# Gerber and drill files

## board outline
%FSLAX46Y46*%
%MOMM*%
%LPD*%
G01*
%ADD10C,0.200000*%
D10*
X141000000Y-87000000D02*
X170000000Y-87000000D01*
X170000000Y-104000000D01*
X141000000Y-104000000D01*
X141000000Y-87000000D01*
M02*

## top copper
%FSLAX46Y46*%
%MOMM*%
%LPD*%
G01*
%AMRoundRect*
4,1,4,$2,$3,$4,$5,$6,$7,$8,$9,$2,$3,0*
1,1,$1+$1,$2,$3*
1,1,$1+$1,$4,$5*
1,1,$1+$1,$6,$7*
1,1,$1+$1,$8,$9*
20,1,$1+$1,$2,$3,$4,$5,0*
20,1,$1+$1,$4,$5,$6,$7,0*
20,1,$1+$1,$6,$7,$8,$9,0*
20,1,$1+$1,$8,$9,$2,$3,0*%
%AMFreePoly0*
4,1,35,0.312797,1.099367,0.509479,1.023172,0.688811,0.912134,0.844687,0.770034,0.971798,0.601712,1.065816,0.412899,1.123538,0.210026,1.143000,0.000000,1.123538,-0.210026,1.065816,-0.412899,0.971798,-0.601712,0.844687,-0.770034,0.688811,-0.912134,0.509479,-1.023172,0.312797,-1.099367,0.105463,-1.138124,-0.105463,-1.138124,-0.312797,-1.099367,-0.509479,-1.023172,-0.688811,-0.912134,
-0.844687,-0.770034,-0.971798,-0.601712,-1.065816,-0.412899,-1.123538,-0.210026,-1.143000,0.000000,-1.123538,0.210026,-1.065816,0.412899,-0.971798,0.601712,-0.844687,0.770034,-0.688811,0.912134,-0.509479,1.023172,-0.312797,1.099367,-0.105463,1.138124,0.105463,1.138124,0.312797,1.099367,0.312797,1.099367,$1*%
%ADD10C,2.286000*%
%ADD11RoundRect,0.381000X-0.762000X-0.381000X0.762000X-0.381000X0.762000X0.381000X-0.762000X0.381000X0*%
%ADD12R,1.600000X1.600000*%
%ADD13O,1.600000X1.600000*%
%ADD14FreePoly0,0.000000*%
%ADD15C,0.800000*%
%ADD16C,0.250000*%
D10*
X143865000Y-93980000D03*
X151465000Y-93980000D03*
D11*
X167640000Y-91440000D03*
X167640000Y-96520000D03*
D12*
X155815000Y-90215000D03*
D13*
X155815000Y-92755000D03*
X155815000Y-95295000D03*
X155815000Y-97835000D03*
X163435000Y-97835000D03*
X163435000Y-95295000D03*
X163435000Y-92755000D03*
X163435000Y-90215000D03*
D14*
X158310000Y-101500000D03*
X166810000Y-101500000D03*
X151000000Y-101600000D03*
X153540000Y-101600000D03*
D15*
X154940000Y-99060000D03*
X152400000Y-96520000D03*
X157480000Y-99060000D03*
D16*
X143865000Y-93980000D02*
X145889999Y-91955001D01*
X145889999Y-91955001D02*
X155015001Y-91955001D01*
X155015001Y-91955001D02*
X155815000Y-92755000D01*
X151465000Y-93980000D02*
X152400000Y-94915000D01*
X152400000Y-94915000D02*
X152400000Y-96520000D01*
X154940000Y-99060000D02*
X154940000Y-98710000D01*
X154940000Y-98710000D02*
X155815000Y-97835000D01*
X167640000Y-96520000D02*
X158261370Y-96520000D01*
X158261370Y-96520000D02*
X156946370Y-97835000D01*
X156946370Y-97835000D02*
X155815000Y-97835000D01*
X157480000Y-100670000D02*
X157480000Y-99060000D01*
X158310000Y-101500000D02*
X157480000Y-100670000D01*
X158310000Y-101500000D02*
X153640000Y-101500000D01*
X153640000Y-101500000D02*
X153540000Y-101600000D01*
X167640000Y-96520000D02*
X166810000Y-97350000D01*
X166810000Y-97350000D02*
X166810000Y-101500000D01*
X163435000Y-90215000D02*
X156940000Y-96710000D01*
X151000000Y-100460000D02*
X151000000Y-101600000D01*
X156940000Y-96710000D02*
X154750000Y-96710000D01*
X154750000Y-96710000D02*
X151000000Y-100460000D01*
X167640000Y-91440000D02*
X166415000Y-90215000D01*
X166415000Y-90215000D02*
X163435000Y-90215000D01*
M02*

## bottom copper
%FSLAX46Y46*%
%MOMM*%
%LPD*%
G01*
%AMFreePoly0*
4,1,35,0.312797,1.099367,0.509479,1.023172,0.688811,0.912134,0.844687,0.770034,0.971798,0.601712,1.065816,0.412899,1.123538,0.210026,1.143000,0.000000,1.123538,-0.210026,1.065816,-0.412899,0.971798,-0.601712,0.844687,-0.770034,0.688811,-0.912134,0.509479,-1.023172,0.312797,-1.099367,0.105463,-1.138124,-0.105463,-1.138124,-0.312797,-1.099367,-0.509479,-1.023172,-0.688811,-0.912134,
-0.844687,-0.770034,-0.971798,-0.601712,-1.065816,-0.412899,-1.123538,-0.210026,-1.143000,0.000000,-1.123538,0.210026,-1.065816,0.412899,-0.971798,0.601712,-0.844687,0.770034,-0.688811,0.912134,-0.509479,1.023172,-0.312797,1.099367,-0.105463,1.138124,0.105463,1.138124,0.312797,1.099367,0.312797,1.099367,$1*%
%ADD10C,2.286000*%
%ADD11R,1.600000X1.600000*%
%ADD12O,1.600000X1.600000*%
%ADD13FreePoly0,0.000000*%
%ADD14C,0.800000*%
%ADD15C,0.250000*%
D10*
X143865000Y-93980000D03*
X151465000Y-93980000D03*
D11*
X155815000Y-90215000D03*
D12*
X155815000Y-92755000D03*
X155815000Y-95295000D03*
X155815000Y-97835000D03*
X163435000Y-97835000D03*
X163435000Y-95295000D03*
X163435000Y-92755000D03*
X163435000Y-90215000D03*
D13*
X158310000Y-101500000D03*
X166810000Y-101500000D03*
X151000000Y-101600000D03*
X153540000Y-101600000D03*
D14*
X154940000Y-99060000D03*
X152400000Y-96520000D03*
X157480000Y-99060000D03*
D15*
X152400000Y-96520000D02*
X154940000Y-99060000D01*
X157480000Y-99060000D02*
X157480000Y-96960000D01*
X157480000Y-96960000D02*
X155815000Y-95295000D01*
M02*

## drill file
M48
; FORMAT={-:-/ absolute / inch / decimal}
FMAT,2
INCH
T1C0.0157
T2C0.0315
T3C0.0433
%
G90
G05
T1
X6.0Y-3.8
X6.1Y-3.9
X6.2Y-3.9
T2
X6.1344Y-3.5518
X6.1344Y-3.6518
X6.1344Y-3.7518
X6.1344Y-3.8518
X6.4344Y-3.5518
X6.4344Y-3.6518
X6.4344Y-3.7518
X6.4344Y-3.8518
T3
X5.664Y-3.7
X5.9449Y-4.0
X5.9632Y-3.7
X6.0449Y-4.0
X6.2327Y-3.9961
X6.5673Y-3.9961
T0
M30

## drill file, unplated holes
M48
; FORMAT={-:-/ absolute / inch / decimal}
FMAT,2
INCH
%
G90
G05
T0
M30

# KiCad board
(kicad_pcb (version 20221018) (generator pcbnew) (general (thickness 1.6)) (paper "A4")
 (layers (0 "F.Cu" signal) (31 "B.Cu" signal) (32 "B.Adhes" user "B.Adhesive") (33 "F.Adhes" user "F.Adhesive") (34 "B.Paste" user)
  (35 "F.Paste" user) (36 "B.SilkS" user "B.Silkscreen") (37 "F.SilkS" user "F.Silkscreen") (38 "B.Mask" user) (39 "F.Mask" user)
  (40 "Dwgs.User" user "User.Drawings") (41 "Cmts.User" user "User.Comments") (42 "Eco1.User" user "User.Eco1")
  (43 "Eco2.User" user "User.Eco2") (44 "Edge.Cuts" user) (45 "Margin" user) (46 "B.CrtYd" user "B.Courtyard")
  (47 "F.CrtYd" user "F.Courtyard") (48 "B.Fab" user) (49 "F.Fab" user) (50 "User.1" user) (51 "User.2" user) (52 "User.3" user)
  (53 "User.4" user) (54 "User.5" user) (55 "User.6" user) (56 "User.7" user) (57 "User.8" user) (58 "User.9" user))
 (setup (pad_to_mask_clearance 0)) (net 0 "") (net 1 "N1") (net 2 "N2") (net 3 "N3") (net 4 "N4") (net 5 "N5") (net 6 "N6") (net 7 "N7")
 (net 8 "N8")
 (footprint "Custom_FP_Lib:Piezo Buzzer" (layer "F.Cu") (at 143.865 93.98)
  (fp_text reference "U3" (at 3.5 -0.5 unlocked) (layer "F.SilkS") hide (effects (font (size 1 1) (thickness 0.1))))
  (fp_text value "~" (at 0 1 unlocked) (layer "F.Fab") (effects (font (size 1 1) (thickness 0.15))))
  (pad "1" thru_hole circle (at 0 0 90) (size 2.286 2.286) (drill 1.1) (layers "*.Cu" "*.Mask") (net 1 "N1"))
  (pad "2" thru_hole circle (at 7.6 0) (size 2.286 2.286) (drill 1.1) (layers "*.Cu" "*.Mask") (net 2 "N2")))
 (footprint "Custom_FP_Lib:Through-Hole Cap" (layer "F.Cu") (at 151 102.87)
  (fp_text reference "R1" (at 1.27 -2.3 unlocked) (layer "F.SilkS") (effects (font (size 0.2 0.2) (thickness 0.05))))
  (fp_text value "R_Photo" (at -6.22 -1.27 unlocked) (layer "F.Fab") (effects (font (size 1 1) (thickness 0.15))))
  (pad "1" thru_hole custom (at 0 -1.27) (size 2.286 2.286) (drill 1.1) (layers "*.Cu" "*.Mask") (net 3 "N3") (thermal_bridge_angle 45)
   (options (clearance outline) (anchor circle)) (primitives))
  (pad "2" thru_hole custom (at 2.54 -1.27) (size 2.286 2.286) (drill 1.1) (layers "*.Cu" "*.Mask") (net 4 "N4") (thermal_bridge_angle 45)
   (options (clearance outline) (anchor circle)) (primitives)))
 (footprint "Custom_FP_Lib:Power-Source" (layer "F.Cu") (at 165.1 93.98)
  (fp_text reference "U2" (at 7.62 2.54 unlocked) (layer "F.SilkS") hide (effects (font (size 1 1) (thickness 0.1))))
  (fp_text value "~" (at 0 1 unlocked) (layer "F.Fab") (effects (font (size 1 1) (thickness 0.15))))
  (pad "1" smd roundrect (at 2.54 -2.54) (size 2.286 1.524) (layers "F.Cu" "F.Paste" "F.Mask") (roundrect_rratio 0.25) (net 3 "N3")
   (thermal_bridge_angle 45))
  (pad "2" smd roundrect (at 2.54 2.54) (size 2.286 1.524) (layers "F.Cu" "F.Paste" "F.Mask") (roundrect_rratio 0.25) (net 2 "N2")
   (thermal_bridge_angle 45)))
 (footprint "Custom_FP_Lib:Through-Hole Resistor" (layer "F.Cu") (at 157.99 102.77)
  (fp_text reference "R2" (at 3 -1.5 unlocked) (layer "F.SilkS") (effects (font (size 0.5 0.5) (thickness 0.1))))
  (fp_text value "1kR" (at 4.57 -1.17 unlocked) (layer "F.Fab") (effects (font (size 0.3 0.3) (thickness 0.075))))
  (pad "1" thru_hole custom (at 0.32 -1.27) (size 2.286 2.286) (drill 1.1) (layers "*.Cu" "*.Mask") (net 4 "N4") (thermal_bridge_angle 45)
   (options (clearance outline) (anchor circle)) (primitives))
  (pad "2" thru_hole custom (at 8.82 -1.27) (size 2.286 2.286) (drill 1.1) (layers "*.Cu" "*.Mask") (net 2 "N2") (thermal_bridge_angle 45)
   (options (clearance outline) (anchor circle)) (primitives)))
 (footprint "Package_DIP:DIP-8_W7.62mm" (layer "F.Cu") (at 155.815 90.215)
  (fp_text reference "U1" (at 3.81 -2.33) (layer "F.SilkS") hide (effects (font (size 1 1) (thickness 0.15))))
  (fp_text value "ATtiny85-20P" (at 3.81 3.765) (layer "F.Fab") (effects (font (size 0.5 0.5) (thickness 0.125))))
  (pad "1" thru_hole rect (at 0 0) (size 1.6 1.6) (drill 0.8) (layers "*.Cu" "*.Mask") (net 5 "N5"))
  (pad "2" thru_hole oval (at 0 2.54) (size 1.6 1.6) (drill 0.8) (layers "*.Cu" "*.Mask") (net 1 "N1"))
  (pad "3" thru_hole oval (at 0 5.08) (size 1.6 1.6) (drill 0.8) (layers "*.Cu" "*.Mask") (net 4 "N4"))
  (pad "4" thru_hole oval (at 0 7.62) (size 1.6 1.6) (drill 0.8) (layers "*.Cu" "*.Mask") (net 2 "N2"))
  (pad "5" thru_hole oval (at 7.62 7.62) (size 1.6 1.6) (drill 0.8) (layers "*.Cu" "*.Mask") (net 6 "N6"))
  (pad "6" thru_hole oval (at 7.62 5.08) (size 1.6 1.6) (drill 0.8) (layers "*.Cu" "*.Mask") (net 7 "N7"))
  (pad "7" thru_hole oval (at 7.62 2.54) (size 1.6 1.6) (drill 0.8) (layers "*.Cu" "*.Mask") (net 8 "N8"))
  (pad "8" thru_hole oval (at 7.62 0) (size 1.6 1.6) (drill 0.8) (layers "*.Cu" "*.Mask") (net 3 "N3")))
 (gr_rect (start 141 87) (end 170 104) (stroke (width 0.2) (type default)) (fill none) (layer "Edge.Cuts"))
 (segment (start 166.415 90.215) (end 163.435 90.215) (width 0.25) (layer "F.Cu") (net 3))
 (segment (start 151 100.46) (end 151 101.6) (width 0.25) (layer "F.Cu") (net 3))
 (segment (start 156.94 96.71) (end 154.75 96.71) (width 0.25) (layer "F.Cu") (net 3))
 (segment (start 163.435 90.215) (end 156.94 96.71) (width 0.25) (layer "F.Cu") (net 3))
 (segment (start 167.64 91.44) (end 166.415 90.215) (width 0.25) (layer "F.Cu") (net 3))
 (segment (start 154.75 96.71) (end 151 100.46) (width 0.25) (layer "F.Cu") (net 3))
 (segment (start 157.48 100.67) (end 157.48 99.06) (width 0.25) (layer "F.Cu") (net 4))
 (segment (start 153.64 101.5) (end 153.54 101.6) (width 0.25) (layer "F.Cu") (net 4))
 (segment (start 158.31 101.5) (end 153.64 101.5) (width 0.25) (layer "F.Cu") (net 4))
 (segment (start 158.31 101.5) (end 157.48 100.67) (width 0.25) (layer "F.Cu") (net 4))
 (via (at 157.48 99.06) (size 0.8) (drill 0.4) (layers "F.Cu" "B.Cu") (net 4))
 (segment (start 157.48 96.96) (end 155.815 95.295) (width 0.25) (layer "B.Cu") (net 4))
 (segment (start 157.48 99.06) (end 157.48 96.96) (width 0.25) (layer "B.Cu") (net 4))
 (segment (start 166.81 97.35) (end 166.81 101.5) (width 0.25) (layer "F.Cu") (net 2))
 (segment (start 167.64 96.52) (end 158.26137 96.52) (width 0.25) (layer "F.Cu") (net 2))
 (segment (start 154.94 99.06) (end 154.94 98.71) (width 0.25) (layer "F.Cu") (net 2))
 (segment (start 152.4 94.915) (end 152.4 96.52) (width 0.25) (layer "F.Cu") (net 2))
 (segment (start 156.94637 97.835) (end 155.815 97.835) (width 0.25) (layer "F.Cu") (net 2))
 (segment (start 154.94 98.71) (end 155.815 97.835) (width 0.25) (layer "F.Cu") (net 2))
 (segment (start 151.465 93.98) (end 152.4 94.915) (width 0.25) (layer "F.Cu") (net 2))
 (segment (start 158.26137 96.52) (end 156.94637 97.835) (width 0.25) (layer "F.Cu") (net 2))
 (segment (start 167.64 96.52) (end 166.81 97.35) (width 0.25) (layer "F.Cu") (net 2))
 (via (at 152.4 96.52) (size 0.8) (drill 0.4) (layers "F.Cu" "B.Cu") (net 2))
 (via (at 154.94 99.06) (size 0.8) (drill 0.4) (layers "F.Cu" "B.Cu") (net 2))
 (segment (start 152.4 96.52) (end 154.94 99.06) (width 0.25) (layer "B.Cu") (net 2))
 (segment (start 155.015001 91.955001) (end 155.815 92.755) (width 0.25) (layer "F.Cu") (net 1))
 (segment (start 145.889999 91.955001) (end 155.015001 91.955001) (width 0.25) (layer "F.Cu") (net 1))
 (segment (start 143.865 93.98) (end 145.889999 91.955001) (width 0.25) (layer "F.Cu") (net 1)))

